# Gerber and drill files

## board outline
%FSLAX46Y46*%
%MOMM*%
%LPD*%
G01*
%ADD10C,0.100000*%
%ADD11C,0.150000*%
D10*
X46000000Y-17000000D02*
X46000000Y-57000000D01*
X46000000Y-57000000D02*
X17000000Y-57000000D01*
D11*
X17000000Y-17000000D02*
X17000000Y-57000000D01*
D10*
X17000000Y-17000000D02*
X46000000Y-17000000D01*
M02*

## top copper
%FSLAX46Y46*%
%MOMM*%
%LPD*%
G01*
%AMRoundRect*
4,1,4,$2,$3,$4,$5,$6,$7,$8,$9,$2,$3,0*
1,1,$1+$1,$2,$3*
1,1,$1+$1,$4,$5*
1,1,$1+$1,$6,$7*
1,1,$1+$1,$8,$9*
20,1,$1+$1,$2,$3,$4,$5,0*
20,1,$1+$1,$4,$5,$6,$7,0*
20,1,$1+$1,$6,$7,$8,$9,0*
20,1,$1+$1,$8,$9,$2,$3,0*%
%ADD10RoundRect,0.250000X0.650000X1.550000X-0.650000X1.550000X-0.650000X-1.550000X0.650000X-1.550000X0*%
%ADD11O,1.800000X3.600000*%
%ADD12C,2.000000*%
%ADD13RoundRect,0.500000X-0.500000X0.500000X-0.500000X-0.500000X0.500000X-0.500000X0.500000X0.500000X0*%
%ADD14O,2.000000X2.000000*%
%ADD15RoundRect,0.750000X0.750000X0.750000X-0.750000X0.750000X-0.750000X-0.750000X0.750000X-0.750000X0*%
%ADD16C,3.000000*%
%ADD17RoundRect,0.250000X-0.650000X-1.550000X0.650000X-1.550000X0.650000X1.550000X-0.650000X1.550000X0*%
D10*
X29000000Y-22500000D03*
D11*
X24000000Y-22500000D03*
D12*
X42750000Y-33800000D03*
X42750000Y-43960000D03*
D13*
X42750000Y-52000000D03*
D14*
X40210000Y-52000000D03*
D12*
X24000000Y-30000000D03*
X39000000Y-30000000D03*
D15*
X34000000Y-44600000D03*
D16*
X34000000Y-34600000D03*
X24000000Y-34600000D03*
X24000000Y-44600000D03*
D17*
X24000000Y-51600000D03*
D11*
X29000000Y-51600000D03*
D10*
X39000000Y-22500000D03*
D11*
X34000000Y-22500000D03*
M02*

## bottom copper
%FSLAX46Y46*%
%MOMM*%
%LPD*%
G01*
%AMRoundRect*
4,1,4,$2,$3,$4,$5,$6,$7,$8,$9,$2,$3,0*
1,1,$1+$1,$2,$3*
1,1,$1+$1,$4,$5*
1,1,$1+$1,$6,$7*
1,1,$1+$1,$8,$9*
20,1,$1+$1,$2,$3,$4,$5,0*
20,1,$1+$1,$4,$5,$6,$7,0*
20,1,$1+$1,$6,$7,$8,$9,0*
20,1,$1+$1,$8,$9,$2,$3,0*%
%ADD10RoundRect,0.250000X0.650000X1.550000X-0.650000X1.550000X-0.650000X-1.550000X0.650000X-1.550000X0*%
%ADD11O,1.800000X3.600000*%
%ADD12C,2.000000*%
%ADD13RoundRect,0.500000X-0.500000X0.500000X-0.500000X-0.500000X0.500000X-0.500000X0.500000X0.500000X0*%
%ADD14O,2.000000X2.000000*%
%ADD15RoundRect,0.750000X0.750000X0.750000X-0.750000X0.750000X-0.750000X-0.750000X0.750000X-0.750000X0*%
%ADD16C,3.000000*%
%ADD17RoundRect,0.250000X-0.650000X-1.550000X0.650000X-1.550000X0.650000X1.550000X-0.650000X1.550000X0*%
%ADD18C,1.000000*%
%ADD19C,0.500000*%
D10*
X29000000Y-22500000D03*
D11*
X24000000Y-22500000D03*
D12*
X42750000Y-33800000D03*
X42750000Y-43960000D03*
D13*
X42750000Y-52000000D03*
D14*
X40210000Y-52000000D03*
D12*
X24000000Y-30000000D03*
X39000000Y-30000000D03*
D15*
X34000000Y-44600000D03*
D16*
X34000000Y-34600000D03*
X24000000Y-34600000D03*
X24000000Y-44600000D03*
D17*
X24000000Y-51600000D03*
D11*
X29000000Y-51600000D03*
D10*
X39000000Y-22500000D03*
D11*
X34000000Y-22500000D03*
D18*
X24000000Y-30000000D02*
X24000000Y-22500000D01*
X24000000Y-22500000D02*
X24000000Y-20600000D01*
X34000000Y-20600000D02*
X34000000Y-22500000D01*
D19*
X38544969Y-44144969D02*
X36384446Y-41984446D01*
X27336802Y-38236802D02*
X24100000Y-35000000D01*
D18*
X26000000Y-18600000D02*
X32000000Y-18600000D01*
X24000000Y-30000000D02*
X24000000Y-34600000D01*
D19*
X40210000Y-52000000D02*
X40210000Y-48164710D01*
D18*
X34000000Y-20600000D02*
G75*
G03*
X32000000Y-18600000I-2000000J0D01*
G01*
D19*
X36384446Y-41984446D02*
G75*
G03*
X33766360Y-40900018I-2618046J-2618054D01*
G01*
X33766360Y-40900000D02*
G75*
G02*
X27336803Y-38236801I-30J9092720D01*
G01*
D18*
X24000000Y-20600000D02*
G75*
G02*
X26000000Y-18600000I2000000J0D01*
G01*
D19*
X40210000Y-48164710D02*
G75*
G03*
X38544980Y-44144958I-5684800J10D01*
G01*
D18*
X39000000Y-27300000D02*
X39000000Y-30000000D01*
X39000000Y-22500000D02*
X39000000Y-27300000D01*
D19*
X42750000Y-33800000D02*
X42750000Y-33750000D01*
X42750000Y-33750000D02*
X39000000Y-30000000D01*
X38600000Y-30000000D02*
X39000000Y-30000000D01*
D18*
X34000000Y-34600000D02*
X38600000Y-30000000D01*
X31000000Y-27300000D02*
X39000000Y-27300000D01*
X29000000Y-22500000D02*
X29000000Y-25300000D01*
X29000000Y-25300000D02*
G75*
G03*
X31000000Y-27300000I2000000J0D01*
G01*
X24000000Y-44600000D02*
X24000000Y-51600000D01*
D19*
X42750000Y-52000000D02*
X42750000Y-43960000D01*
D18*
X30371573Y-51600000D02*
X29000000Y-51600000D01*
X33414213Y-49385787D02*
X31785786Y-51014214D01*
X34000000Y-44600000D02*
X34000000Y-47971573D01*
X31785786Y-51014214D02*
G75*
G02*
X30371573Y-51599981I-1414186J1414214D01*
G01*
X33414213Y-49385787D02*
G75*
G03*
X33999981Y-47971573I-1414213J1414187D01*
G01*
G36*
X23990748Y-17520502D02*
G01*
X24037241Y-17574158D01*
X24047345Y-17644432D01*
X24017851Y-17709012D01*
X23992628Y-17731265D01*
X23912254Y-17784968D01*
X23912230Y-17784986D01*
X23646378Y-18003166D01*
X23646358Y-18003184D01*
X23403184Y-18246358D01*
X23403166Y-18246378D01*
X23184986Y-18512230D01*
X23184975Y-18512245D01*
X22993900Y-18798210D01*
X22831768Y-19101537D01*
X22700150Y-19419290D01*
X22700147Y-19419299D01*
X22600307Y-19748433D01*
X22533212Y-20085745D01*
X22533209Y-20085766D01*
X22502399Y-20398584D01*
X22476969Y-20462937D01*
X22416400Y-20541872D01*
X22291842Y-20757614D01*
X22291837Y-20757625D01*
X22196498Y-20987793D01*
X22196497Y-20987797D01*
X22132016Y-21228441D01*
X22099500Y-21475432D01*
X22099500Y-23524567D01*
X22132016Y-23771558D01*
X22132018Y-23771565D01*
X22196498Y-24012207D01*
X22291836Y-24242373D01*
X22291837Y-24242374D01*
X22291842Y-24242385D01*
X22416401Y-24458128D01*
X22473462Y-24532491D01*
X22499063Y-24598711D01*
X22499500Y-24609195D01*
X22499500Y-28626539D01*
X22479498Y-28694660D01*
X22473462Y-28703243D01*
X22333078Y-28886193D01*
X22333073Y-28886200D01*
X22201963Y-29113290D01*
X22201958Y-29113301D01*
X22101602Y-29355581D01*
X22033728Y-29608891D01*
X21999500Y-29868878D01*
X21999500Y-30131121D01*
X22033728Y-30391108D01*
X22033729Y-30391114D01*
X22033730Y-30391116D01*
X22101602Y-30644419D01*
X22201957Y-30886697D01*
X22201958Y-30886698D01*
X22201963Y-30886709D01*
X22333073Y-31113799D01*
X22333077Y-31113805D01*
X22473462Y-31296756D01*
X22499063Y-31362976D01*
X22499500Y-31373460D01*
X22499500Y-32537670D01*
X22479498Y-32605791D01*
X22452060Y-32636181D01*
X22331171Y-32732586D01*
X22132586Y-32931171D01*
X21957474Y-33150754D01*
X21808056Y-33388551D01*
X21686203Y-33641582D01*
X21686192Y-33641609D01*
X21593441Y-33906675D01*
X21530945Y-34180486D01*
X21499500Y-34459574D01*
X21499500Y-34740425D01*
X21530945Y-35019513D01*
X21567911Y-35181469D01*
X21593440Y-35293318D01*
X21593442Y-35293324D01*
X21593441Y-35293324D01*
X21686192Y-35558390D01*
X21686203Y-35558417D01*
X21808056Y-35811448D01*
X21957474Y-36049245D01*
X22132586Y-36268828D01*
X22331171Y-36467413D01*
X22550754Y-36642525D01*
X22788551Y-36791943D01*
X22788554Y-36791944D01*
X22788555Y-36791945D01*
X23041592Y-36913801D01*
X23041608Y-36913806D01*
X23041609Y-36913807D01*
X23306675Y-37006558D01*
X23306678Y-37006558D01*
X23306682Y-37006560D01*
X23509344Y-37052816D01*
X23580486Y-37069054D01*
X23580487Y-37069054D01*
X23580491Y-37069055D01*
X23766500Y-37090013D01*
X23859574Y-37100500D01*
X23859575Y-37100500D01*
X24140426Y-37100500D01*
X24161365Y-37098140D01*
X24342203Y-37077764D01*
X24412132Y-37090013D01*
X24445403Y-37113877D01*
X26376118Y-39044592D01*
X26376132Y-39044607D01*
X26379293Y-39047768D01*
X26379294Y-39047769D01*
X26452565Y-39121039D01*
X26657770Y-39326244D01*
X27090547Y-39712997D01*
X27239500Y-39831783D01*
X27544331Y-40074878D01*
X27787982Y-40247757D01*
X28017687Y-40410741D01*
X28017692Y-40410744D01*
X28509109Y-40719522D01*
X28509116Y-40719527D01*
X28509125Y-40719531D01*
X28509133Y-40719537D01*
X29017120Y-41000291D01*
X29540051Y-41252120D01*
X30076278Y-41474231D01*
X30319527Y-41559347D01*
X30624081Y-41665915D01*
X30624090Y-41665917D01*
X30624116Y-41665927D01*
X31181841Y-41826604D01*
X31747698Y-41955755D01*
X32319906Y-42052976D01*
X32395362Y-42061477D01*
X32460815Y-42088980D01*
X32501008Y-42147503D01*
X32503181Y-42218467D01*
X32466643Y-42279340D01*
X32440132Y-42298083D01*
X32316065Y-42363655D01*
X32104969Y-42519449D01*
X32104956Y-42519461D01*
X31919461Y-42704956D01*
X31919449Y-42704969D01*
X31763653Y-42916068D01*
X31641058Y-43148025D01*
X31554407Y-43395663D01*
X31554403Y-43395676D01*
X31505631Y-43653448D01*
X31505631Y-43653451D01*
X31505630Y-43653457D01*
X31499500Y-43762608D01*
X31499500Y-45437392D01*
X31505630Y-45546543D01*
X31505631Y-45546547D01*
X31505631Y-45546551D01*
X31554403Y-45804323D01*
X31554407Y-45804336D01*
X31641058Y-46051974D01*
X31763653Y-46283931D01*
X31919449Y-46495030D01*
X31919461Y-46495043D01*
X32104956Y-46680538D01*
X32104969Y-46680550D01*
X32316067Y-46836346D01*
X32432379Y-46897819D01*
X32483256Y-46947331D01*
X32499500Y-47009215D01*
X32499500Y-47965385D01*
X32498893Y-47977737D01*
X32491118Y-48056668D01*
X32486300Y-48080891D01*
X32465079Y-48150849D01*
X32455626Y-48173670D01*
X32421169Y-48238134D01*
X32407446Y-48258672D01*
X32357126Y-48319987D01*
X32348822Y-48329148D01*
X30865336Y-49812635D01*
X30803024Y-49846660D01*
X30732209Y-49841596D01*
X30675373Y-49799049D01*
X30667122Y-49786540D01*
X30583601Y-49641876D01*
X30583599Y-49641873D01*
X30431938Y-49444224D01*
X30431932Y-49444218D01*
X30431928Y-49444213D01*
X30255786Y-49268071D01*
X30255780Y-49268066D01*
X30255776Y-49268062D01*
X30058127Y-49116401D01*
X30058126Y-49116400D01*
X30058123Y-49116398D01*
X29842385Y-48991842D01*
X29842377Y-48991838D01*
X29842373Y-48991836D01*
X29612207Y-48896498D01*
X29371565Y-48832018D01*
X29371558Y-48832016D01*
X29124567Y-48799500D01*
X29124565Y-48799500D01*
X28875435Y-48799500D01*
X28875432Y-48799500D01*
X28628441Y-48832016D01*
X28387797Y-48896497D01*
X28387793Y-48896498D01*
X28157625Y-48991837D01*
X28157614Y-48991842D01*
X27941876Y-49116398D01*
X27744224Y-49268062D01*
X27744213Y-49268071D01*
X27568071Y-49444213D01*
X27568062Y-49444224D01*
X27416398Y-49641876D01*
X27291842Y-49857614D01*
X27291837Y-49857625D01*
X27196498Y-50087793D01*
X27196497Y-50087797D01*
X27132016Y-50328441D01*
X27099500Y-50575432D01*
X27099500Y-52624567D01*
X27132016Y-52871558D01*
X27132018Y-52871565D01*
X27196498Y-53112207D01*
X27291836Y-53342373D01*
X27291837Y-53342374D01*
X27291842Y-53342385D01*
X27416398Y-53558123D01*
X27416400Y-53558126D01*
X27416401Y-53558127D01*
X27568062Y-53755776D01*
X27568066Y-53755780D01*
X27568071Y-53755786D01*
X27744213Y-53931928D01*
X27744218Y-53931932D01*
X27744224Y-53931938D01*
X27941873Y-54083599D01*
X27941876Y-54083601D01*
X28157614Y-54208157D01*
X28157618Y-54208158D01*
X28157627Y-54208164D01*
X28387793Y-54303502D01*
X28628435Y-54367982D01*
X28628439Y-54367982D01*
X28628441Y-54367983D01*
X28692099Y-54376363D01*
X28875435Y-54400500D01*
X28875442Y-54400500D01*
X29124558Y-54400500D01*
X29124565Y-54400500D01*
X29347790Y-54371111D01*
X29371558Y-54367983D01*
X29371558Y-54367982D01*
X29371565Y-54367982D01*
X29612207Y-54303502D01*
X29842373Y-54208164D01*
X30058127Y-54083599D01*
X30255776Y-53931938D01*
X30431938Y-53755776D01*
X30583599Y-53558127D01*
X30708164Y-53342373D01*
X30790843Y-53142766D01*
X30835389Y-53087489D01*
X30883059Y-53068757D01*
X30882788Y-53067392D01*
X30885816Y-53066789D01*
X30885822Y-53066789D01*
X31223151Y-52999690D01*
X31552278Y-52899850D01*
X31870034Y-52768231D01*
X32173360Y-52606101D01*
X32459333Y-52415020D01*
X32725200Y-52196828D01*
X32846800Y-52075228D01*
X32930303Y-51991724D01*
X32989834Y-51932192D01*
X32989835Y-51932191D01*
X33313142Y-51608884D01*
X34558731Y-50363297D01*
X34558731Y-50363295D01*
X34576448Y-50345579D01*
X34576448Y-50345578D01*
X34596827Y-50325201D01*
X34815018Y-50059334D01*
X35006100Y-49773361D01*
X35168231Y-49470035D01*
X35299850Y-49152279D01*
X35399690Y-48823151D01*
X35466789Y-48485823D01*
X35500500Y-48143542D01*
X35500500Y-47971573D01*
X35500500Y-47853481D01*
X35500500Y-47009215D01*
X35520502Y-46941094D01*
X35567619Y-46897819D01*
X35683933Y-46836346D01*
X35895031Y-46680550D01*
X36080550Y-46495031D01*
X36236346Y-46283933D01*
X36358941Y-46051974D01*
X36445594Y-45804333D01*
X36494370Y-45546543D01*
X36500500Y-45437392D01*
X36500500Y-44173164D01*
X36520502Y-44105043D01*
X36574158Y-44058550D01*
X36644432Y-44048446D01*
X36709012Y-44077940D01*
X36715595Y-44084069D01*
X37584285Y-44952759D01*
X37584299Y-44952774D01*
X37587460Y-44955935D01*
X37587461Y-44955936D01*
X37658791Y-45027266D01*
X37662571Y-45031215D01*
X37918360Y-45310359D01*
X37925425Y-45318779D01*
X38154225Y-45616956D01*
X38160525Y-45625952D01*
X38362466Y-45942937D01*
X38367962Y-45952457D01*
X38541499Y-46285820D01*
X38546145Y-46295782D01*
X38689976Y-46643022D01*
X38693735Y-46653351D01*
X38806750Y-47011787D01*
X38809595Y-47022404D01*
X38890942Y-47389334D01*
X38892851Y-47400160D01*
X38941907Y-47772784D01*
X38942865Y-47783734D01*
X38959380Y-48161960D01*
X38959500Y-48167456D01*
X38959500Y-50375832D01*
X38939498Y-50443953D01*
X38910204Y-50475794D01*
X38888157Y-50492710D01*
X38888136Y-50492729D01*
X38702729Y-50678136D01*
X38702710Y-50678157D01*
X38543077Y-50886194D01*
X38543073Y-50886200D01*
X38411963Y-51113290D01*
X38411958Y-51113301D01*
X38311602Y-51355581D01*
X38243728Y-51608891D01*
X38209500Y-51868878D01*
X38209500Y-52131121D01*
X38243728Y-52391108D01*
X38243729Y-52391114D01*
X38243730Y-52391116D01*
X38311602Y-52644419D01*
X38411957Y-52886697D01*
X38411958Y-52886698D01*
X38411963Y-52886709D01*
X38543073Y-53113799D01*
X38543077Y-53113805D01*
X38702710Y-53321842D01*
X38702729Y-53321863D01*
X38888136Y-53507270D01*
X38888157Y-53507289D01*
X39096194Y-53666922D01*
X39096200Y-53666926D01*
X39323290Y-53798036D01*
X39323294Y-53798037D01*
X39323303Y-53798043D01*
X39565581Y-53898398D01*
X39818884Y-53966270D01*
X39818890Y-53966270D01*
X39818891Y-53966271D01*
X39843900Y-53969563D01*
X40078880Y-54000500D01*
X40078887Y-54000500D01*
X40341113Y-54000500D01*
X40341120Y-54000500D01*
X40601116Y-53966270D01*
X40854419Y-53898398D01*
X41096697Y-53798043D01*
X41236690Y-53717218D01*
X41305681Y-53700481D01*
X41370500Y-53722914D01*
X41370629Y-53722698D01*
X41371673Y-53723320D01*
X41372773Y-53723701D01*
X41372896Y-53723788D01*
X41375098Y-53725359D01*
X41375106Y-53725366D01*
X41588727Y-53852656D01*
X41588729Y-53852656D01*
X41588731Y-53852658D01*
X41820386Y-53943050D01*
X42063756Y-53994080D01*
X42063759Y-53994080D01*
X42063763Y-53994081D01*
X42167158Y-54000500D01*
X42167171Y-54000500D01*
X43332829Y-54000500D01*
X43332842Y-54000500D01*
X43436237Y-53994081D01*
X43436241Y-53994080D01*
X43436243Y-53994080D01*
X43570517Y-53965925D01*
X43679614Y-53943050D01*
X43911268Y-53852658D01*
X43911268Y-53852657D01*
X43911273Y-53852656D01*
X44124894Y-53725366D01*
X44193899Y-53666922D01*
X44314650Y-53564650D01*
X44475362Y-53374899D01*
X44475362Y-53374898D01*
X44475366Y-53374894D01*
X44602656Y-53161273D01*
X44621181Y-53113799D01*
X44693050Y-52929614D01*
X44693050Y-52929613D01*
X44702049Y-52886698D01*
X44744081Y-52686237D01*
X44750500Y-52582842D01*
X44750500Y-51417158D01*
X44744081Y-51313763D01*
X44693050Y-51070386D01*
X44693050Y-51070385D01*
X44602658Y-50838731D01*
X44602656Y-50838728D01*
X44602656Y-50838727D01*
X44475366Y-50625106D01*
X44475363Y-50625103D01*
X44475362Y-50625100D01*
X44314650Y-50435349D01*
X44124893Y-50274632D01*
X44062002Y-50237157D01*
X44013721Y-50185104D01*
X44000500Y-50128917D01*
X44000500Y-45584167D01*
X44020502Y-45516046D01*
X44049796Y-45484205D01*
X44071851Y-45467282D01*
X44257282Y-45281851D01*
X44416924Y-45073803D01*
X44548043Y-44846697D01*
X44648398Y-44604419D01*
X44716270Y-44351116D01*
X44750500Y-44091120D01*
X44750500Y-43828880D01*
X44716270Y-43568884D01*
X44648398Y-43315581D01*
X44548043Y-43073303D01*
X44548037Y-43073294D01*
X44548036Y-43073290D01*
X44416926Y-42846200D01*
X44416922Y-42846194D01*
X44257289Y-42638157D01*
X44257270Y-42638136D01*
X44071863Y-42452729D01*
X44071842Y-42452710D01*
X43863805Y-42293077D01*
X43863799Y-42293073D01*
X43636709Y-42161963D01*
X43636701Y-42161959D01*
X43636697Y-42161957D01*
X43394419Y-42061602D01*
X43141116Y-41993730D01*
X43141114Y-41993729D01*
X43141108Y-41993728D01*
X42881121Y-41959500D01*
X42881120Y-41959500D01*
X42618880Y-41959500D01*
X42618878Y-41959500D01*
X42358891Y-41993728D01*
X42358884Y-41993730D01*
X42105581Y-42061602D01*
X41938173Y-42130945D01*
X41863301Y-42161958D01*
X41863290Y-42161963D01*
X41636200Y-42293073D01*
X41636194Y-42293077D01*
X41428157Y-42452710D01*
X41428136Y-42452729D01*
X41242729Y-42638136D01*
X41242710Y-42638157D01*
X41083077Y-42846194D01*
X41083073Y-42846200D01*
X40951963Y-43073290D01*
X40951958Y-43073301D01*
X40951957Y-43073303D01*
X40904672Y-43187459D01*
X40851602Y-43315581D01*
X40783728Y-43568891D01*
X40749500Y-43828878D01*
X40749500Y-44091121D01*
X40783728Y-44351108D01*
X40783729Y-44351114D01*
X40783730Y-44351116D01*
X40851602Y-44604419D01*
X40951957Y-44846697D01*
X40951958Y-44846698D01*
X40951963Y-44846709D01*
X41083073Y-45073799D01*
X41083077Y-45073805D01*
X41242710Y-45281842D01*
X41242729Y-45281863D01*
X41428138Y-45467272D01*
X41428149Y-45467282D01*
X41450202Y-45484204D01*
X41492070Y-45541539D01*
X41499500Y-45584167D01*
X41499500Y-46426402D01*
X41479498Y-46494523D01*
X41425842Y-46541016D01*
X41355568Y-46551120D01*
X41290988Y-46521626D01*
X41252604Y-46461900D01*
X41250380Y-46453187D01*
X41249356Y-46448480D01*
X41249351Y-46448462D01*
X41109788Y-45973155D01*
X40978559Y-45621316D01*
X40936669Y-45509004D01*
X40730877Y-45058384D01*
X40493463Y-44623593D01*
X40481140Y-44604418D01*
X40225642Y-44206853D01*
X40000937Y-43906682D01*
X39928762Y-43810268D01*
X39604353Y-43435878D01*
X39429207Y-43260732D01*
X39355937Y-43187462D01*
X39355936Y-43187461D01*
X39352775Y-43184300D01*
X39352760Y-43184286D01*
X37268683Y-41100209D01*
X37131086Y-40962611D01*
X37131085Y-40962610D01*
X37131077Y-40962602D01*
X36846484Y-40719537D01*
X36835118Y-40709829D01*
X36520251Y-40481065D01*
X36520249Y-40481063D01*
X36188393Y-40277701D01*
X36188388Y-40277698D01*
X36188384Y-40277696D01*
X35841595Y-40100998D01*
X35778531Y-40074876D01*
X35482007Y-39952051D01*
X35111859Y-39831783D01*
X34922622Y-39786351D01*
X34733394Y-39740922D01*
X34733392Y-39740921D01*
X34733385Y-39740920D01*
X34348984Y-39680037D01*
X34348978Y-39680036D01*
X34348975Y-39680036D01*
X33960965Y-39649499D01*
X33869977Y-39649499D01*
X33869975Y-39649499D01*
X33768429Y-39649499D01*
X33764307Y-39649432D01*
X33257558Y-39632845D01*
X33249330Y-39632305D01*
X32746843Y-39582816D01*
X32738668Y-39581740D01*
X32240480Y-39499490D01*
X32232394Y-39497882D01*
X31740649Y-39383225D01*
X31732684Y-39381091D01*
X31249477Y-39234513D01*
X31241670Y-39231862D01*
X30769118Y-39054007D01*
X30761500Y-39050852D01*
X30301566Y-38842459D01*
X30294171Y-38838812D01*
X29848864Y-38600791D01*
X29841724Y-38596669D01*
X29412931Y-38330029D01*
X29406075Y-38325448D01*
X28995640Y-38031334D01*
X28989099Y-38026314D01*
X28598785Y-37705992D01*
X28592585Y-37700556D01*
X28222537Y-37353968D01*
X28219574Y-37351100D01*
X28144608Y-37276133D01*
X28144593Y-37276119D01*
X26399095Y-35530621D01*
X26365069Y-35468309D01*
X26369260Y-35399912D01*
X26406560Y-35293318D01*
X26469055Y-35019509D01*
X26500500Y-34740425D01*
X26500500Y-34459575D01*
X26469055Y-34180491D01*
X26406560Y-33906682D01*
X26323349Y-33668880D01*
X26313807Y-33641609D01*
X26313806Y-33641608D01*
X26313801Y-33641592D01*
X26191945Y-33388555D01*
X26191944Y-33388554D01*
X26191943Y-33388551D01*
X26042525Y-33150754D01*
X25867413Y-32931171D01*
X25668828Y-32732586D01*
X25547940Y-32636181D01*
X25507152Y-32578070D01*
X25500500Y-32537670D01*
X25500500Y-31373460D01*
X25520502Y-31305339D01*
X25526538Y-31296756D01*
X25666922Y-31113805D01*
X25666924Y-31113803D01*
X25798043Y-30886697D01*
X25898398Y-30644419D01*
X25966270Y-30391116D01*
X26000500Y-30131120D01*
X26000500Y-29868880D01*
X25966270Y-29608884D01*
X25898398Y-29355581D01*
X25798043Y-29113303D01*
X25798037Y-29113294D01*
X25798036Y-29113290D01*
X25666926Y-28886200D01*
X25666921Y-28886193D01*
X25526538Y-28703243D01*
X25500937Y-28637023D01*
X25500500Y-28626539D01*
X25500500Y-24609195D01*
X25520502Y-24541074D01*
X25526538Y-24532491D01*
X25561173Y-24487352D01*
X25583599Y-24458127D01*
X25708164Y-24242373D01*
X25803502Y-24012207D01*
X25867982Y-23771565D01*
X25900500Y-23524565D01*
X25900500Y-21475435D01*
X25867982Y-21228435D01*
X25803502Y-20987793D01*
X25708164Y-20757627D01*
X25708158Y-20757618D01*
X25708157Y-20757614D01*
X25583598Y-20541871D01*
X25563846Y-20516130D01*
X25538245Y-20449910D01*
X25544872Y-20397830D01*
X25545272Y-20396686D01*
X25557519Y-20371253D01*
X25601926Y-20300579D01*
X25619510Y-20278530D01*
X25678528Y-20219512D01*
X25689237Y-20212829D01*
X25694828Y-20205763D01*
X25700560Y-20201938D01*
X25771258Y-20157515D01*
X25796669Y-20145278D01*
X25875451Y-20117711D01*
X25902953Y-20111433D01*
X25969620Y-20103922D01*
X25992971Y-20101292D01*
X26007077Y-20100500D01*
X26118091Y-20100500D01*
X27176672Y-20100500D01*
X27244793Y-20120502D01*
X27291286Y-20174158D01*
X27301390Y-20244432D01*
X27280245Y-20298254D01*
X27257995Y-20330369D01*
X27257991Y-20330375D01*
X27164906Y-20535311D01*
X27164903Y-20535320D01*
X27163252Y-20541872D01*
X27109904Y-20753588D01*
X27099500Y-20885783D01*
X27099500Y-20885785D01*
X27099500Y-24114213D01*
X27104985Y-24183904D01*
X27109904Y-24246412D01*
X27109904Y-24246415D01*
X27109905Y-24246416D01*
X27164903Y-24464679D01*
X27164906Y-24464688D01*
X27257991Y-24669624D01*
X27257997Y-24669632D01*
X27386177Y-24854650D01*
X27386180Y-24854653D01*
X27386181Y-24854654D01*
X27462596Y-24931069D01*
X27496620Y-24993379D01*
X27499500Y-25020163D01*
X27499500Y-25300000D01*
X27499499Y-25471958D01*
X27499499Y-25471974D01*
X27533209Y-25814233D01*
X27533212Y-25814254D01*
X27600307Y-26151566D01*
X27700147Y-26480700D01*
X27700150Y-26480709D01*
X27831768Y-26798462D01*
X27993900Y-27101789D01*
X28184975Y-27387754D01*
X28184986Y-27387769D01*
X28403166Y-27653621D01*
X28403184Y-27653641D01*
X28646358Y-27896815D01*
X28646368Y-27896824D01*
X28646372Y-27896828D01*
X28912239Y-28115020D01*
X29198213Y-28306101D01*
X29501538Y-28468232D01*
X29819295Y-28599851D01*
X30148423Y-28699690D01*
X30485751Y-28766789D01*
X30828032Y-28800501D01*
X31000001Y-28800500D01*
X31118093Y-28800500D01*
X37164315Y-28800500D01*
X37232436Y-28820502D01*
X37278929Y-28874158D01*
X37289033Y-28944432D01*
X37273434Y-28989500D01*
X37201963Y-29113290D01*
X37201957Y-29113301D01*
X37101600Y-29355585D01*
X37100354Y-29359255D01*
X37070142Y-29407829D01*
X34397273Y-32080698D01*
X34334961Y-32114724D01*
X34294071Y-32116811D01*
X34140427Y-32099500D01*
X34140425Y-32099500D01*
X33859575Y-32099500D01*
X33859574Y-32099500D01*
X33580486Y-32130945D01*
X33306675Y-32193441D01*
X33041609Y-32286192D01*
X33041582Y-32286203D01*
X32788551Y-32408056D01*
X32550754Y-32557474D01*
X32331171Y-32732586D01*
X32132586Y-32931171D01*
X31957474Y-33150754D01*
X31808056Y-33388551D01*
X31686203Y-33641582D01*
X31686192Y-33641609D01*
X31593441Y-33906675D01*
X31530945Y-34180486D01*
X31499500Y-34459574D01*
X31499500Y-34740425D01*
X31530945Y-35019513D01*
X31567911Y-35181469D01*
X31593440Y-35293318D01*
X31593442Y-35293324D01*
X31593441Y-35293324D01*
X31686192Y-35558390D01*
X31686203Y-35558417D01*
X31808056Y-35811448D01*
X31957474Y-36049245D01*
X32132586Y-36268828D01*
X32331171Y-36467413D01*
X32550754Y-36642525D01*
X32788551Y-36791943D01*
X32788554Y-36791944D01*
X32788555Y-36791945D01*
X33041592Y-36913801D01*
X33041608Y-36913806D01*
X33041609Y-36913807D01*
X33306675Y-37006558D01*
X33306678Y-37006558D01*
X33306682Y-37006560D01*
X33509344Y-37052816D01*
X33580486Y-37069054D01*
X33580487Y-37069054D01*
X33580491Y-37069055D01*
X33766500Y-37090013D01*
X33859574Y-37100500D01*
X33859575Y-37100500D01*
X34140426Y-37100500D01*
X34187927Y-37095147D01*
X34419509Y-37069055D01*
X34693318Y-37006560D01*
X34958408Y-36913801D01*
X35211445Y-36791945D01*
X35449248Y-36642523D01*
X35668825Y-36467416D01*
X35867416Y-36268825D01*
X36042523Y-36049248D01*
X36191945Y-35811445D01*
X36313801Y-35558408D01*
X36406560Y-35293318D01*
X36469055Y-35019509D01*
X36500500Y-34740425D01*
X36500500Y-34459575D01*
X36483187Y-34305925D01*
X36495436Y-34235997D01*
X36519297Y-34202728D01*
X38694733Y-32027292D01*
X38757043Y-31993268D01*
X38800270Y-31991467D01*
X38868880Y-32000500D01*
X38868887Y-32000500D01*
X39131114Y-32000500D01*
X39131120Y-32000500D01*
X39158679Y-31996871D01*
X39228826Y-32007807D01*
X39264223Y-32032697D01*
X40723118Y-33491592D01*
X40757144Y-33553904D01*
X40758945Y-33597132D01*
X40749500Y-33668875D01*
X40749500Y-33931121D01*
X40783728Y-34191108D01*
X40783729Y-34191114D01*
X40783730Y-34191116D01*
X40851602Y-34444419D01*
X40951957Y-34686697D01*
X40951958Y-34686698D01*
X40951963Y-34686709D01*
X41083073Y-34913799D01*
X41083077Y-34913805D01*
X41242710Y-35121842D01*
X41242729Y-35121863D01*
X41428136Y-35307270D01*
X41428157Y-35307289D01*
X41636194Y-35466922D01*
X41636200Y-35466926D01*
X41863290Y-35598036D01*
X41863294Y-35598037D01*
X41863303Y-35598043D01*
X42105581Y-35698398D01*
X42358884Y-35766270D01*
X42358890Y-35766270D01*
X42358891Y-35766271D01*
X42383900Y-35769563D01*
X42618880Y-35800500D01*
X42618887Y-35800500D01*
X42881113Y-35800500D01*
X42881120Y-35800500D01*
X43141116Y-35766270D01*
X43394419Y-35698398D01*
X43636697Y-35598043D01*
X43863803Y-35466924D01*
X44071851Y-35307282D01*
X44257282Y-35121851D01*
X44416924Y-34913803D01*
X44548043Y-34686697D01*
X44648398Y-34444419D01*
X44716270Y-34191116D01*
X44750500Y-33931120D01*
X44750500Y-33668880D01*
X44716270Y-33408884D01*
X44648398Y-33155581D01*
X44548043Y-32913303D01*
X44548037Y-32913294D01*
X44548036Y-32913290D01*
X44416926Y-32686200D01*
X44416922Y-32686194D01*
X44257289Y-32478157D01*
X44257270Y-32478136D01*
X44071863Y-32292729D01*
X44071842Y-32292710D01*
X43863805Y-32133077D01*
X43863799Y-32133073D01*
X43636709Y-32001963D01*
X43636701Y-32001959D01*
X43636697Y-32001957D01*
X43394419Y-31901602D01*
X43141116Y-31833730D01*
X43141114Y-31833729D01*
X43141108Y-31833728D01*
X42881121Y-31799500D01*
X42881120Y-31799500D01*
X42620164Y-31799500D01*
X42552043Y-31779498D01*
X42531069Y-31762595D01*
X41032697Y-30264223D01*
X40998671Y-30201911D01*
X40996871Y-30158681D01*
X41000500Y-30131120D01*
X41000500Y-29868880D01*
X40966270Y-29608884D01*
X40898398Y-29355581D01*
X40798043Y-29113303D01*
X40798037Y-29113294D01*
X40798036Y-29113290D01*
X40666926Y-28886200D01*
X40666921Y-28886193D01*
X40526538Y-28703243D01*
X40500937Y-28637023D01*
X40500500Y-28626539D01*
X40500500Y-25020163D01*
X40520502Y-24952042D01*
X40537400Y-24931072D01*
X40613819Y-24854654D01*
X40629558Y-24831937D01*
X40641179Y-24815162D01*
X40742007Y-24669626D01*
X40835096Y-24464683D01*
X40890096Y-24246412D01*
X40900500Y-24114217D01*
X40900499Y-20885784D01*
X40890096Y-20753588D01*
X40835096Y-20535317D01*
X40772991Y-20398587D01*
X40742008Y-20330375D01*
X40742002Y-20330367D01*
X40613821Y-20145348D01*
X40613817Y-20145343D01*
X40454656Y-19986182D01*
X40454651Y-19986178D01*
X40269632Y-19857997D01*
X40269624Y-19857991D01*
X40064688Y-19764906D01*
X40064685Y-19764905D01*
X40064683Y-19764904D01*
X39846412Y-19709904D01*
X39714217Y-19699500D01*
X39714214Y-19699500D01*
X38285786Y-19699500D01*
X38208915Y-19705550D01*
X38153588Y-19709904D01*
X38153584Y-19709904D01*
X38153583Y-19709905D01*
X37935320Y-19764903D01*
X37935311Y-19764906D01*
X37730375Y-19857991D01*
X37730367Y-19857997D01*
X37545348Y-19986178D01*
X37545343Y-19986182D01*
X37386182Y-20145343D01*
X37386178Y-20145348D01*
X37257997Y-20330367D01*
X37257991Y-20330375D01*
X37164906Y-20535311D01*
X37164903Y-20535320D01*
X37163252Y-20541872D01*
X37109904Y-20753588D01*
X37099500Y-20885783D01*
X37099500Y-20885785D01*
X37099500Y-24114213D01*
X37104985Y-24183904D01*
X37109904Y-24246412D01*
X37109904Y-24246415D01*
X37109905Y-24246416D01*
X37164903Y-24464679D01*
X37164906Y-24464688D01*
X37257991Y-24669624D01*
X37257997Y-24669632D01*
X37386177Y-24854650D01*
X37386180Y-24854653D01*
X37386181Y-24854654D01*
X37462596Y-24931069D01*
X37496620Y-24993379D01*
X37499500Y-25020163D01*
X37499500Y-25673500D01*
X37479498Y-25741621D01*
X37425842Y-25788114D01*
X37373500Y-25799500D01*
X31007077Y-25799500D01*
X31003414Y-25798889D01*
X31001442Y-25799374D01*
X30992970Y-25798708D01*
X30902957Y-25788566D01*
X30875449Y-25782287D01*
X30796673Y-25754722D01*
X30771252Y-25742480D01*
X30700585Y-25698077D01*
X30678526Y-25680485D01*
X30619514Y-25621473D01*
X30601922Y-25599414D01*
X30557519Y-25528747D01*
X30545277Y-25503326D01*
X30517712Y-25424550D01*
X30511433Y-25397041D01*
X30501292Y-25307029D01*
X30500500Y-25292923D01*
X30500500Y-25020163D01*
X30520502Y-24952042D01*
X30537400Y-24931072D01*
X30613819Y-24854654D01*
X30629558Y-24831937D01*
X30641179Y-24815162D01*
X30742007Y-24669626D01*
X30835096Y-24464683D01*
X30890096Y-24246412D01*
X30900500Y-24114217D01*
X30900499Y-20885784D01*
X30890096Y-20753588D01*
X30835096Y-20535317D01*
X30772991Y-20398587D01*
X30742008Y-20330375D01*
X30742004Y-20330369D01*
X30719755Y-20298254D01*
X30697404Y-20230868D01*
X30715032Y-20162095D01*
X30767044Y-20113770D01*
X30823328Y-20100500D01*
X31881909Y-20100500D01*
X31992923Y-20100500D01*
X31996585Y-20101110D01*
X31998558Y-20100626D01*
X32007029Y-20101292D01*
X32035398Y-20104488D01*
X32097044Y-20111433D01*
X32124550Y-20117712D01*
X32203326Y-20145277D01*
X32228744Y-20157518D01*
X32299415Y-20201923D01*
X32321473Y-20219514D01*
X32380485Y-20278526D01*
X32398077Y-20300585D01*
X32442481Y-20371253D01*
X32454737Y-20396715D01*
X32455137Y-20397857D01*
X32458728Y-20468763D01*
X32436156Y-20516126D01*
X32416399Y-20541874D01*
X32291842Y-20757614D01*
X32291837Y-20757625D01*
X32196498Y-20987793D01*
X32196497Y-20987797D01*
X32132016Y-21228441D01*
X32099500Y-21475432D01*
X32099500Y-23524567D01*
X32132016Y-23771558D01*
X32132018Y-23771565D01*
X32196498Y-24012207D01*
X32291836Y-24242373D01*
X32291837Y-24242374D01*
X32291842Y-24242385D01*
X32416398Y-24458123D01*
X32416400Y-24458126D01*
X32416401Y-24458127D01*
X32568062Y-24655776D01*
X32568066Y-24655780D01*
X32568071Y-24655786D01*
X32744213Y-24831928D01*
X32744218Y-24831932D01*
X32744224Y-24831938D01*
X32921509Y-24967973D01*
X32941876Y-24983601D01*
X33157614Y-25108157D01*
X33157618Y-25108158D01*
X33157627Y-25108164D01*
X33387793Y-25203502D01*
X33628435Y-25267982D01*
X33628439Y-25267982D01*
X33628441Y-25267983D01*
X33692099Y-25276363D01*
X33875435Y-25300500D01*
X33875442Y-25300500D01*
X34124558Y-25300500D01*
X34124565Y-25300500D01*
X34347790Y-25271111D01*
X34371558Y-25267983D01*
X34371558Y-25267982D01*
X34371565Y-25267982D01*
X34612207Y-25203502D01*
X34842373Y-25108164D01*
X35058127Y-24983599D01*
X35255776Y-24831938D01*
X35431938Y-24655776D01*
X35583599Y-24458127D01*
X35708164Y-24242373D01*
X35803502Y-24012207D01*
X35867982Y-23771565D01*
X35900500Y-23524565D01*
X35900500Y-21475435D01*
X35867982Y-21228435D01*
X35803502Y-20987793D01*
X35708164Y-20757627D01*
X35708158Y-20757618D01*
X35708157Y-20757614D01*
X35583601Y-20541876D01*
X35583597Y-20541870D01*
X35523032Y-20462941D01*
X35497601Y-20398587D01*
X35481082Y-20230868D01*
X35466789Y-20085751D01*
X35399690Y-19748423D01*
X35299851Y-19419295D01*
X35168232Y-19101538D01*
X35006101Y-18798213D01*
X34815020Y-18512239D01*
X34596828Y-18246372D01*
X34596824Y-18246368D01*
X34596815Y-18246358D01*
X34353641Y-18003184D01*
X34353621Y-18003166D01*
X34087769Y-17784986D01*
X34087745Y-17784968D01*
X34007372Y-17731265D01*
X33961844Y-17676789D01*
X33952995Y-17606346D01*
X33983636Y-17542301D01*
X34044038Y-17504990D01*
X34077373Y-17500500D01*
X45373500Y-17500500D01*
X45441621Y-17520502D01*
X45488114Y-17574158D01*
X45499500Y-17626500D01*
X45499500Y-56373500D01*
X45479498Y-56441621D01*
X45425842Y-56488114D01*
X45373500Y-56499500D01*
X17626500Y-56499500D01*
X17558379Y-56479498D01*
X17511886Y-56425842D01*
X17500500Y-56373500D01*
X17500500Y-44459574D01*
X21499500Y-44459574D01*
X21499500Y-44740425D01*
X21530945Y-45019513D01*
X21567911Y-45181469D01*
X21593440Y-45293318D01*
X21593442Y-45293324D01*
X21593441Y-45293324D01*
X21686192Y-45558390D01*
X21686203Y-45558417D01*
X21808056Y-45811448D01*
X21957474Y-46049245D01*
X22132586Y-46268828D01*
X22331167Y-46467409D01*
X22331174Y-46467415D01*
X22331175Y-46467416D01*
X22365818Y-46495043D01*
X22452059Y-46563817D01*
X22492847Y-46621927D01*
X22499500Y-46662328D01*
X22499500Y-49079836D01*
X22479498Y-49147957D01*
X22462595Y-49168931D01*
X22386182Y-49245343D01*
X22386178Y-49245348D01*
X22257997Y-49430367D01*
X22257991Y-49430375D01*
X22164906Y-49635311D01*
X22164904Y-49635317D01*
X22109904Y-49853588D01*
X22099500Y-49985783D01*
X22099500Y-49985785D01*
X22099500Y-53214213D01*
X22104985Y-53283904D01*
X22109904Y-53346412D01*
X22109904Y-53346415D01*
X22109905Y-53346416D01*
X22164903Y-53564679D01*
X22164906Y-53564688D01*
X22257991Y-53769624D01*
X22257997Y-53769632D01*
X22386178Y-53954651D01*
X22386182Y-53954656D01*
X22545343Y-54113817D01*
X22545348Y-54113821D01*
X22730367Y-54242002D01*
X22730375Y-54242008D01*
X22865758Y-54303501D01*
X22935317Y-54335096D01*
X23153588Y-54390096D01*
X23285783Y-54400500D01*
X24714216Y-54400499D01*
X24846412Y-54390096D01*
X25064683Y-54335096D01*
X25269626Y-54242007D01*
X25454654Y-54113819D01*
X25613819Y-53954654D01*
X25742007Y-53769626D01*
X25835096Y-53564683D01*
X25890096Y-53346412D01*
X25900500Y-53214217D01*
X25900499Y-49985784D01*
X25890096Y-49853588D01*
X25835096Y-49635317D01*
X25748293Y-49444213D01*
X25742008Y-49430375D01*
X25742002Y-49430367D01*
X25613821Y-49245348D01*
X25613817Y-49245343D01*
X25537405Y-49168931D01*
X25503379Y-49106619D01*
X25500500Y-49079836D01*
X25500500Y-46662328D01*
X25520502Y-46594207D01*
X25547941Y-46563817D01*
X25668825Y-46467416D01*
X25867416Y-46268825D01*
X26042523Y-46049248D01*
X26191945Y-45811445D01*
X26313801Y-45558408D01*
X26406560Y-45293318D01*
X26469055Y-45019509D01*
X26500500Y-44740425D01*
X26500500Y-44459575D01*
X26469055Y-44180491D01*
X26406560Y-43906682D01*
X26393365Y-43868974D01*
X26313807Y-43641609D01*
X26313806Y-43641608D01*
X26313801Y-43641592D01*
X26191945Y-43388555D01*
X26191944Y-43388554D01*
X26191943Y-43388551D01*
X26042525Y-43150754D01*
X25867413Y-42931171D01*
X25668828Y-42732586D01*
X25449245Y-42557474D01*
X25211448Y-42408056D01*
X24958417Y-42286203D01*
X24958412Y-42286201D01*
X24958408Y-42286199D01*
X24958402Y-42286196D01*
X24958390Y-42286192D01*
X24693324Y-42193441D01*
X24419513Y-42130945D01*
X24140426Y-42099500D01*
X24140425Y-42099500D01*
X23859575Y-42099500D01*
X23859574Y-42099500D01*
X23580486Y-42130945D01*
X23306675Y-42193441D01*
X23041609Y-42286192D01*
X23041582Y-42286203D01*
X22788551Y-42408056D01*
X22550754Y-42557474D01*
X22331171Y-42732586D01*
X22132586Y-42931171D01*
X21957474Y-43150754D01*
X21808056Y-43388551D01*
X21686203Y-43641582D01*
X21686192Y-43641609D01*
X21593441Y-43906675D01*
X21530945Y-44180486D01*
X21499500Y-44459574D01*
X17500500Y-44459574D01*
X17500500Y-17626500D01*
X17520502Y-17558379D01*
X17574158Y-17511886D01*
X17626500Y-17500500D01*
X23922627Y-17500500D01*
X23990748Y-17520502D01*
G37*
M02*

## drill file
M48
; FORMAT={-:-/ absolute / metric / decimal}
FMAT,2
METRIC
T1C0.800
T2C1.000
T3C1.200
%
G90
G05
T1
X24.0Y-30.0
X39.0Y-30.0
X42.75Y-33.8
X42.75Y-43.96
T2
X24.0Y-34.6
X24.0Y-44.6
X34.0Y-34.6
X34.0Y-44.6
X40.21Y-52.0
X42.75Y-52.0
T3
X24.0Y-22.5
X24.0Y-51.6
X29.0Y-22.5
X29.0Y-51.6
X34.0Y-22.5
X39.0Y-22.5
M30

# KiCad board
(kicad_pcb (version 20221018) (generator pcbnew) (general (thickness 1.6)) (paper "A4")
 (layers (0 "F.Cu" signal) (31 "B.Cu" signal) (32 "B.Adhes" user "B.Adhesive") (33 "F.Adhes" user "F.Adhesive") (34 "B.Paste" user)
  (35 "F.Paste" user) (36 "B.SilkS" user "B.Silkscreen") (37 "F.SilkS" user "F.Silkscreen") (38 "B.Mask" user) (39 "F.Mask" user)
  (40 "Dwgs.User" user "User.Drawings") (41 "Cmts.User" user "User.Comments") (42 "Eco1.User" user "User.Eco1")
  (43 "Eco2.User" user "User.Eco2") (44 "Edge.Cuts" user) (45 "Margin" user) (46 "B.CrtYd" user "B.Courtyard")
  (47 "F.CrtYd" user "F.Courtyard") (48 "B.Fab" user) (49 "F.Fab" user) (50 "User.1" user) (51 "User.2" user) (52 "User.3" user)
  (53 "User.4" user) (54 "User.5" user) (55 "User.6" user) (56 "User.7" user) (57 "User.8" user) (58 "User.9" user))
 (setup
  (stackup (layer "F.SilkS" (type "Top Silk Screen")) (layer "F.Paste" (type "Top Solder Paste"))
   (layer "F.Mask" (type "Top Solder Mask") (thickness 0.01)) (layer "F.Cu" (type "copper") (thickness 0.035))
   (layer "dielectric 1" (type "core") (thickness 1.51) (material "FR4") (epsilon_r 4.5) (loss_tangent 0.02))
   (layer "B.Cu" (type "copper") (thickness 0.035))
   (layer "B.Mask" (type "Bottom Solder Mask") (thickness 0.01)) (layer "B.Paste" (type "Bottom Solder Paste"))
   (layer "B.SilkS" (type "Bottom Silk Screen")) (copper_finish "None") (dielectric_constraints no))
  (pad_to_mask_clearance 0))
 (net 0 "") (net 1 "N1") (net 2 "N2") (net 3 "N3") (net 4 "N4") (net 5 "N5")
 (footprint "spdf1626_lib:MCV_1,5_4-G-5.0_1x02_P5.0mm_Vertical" (layer "F.Cu") (at 26.5 22.5 180)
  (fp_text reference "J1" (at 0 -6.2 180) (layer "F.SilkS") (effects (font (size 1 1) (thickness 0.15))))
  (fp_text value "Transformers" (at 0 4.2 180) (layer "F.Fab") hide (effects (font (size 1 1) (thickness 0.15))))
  (pad "1" thru_hole roundrect (at -2.5 0 180) (size 1.8 3.6) (drill 1.2) (layers "*.Cu" "*.Mask") (roundrect_rratio 0.138889) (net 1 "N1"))
  (pad "2" thru_hole oval (at 2.5 0 180) (size 1.8 3.6) (drill 1.2) (layers "*.Cu" "*.Mask") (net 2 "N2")))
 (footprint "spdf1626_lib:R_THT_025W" (layer "F.Cu") (at 42.75 33.8 -90)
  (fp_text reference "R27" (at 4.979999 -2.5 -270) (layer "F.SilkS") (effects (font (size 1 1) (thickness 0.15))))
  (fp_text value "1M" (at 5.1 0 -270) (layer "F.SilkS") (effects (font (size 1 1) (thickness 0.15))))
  (pad "1" thru_hole circle (at 0 0 270) (size 2 2) (drill 0.8) (layers "*.Cu" "*.Mask") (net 1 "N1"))
  (pad "2" thru_hole circle (at 10.16 0 270) (size 2 2) (drill 0.8) (layers "*.Cu" "*.Mask") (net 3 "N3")))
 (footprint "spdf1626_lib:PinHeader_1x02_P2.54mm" (layer "F.Cu") (at 42.75 52 -90)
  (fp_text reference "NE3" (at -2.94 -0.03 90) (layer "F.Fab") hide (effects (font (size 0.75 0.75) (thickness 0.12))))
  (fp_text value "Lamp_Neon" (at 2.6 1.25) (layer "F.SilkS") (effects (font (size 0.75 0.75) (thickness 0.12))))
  (pad "1" thru_hole roundrect (at 0 0 270) (size 2 2) (drill 1) (layers "*.Cu" "*.Mask") (roundrect_rratio 0.25) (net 3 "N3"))
  (pad "2" thru_hole oval (at 0 2.54 270) (size 2 2) (drill 1) (layers "*.Cu" "*.Mask") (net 2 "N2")))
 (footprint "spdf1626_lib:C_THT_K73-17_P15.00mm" (layer "F.Cu") (at 31.5 30)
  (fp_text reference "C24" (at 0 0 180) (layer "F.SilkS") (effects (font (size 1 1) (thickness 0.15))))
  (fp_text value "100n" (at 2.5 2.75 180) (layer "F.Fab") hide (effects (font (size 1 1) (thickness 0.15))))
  (pad "1" thru_hole circle (at -7.5 0) (size 2 2) (drill 0.8) (layers "*.Cu" "*.Mask") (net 2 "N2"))
  (pad "2" thru_hole circle (at 7.5 0) (size 2 2) (drill 0.8) (layers "*.Cu" "*.Mask") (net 1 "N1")))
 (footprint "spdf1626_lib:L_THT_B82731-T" (layer "F.Cu") (at 29 39.6 180)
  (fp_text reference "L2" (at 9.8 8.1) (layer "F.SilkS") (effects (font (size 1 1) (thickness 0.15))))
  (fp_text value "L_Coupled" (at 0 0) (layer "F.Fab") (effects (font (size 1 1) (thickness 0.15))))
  (pad "1" thru_hole roundrect (at -5 -5 180) (size 3 3) (drill 1) (layers "*.Cu" "*.Mask") (roundrect_rratio 0.25) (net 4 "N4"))
  (pad "2" thru_hole circle (at -5 5 180) (size 3 3) (drill 1) (layers "*.Cu" "*.Mask") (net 1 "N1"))
  (pad "3" thru_hole circle (at 5 5 180) (size 3 3) (drill 1) (layers "*.Cu" "*.Mask") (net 2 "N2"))
  (pad "4" thru_hole circle (at 5 -5 180) (size 3 3) (drill 1) (layers "*.Cu" "*.Mask") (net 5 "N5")))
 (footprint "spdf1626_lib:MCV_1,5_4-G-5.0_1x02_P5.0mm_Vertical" (layer "F.Cu") (at 26.5 51.6)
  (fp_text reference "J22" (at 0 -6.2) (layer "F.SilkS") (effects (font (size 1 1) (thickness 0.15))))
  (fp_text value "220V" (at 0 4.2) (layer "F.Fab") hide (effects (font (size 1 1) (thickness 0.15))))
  (pad "1" thru_hole roundrect (at -2.5 0) (size 1.8 3.6) (drill 1.2) (layers "*.Cu" "*.Mask") (roundrect_rratio 0.138889) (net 5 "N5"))
  (pad "2" thru_hole oval (at 2.5 0) (size 1.8 3.6) (drill 1.2) (layers "*.Cu" "*.Mask") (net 4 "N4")))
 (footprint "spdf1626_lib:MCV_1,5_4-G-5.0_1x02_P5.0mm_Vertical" (layer "F.Cu") (at 36.5 22.5 180)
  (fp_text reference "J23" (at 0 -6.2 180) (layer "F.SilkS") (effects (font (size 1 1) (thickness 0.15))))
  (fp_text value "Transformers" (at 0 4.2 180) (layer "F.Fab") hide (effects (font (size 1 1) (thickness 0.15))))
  (pad "1" thru_hole roundrect (at -2.5 0 180) (size 1.8 3.6) (drill 1.2) (layers "*.Cu" "*.Mask") (roundrect_rratio 0.138889) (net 1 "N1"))
  (pad "2" thru_hole oval (at 2.5 0 180) (size 1.8 3.6) (drill 1.2) (layers "*.Cu" "*.Mask") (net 2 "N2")))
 (gr_line (start 46 17) (end 46 57) (stroke (width 0.1) (type default)) (layer "Edge.Cuts"))
 (gr_line (start 46 57) (end 17 57) (stroke (width 0.1) (type default)) (layer "Edge.Cuts"))
 (gr_line (start 17 17) (end 17 57) (stroke (width 0.15) (type solid)) (layer "Edge.Cuts"))
 (gr_line (start 17 17) (end 46 17) (stroke (width 0.1) (type default)) (layer "Edge.Cuts"))
 (segment (start 24 30) (end 24 22.5) (width 1) (layer "B.Cu") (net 2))
 (segment (start 24 22.5) (end 24 20.6) (width 1) (layer "B.Cu") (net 2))
 (segment (start 34 20.6) (end 34 22.5) (width 1) (layer "B.Cu") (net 2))
 (segment (start 38.544969 44.144969) (end 36.384446 41.984446) (width 0.5) (layer "B.Cu") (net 2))
 (segment (start 27.336802 38.236802) (end 24.1 35) (width 0.5) (layer "B.Cu") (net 2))
 (segment (start 26 18.6) (end 32 18.6) (width 1) (layer "B.Cu") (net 2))
 (segment (start 24 30) (end 24 34.6) (width 1) (layer "B.Cu") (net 2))
 (segment (start 40.21 52) (end 40.21 48.16471) (width 0.5) (layer "B.Cu") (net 2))
 (arc (start 34 20.6) (mid 33.414214 19.185786) (end 32 18.6) (width 1) (layer "B.Cu") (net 2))
 (arc (start 36.384446 41.984446) (mid 35.183258 41.181838) (end 33.76636 40.9) (width 0.5) (layer "B.Cu") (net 2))
 (arc (start 33.76636 40.9) (mid 30.286694 40.207858) (end 27.336802 38.236802) (width 0.5) (layer "B.Cu") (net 2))
 (arc (start 24 20.6) (mid 24.585786 19.185786) (end 26 18.6) (width 1) (layer "B.Cu") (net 2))
 (arc (start 40.21 48.16471) (mid 39.777272 45.989242) (end 38.544969 44.144969) (width 0.5) (layer "B.Cu") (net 2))
 (segment (start 39 27.3) (end 39 30) (width 1) (layer "B.Cu") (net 1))
 (segment (start 39 22.5) (end 39 27.3) (width 1) (layer "B.Cu") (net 1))
 (segment (start 42.75 33.8) (end 42.75 33.75) (width 0.5) (layer "B.Cu") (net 1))
 (segment (start 42.75 33.75) (end 39 30) (width 0.5) (layer "B.Cu") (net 1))
 (segment (start 38.6 30) (end 39 30) (width 0.5) (layer "B.Cu") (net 1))
 (segment (start 34 34.6) (end 38.6 30) (width 1) (layer "B.Cu") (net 1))
 (segment (start 31 27.3) (end 39 27.3) (width 1) (layer "B.Cu") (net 1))
 (segment (start 29 22.5) (end 29 25.3) (width 1) (layer "B.Cu") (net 1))
 (arc (start 29 25.3) (mid 29.585786 26.714214) (end 31 27.3) (width 1) (layer "B.Cu") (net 1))
 (segment (start 24 44.6) (end 24 51.6) (width 1) (layer "B.Cu") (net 5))
 (segment (start 42.75 52) (end 42.75 43.96) (width 0.5) (layer "B.Cu") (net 3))
 (segment (start 30.371573 51.6) (end 29 51.6) (width 1) (layer "B.Cu") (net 4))
 (segment (start 33.414213 49.385787) (end 31.785786 51.014214) (width 1) (layer "B.Cu") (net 4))
 (segment (start 34 44.6) (end 34 47.971573) (width 1) (layer "B.Cu") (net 4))
 (arc (start 31.785786 51.014214) (mid 31.13694 51.447759) (end 30.371573 51.6) (width 1) (layer "B.Cu") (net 4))
 (arc (start 33.414213 49.385787) (mid 33.847759 48.73694) (end 34 47.971573) (width 1) (layer "B.Cu") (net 4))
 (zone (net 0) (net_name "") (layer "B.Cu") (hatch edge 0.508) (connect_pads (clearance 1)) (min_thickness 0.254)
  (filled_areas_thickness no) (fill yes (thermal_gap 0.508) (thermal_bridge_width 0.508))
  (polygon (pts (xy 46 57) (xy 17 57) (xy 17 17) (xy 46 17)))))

